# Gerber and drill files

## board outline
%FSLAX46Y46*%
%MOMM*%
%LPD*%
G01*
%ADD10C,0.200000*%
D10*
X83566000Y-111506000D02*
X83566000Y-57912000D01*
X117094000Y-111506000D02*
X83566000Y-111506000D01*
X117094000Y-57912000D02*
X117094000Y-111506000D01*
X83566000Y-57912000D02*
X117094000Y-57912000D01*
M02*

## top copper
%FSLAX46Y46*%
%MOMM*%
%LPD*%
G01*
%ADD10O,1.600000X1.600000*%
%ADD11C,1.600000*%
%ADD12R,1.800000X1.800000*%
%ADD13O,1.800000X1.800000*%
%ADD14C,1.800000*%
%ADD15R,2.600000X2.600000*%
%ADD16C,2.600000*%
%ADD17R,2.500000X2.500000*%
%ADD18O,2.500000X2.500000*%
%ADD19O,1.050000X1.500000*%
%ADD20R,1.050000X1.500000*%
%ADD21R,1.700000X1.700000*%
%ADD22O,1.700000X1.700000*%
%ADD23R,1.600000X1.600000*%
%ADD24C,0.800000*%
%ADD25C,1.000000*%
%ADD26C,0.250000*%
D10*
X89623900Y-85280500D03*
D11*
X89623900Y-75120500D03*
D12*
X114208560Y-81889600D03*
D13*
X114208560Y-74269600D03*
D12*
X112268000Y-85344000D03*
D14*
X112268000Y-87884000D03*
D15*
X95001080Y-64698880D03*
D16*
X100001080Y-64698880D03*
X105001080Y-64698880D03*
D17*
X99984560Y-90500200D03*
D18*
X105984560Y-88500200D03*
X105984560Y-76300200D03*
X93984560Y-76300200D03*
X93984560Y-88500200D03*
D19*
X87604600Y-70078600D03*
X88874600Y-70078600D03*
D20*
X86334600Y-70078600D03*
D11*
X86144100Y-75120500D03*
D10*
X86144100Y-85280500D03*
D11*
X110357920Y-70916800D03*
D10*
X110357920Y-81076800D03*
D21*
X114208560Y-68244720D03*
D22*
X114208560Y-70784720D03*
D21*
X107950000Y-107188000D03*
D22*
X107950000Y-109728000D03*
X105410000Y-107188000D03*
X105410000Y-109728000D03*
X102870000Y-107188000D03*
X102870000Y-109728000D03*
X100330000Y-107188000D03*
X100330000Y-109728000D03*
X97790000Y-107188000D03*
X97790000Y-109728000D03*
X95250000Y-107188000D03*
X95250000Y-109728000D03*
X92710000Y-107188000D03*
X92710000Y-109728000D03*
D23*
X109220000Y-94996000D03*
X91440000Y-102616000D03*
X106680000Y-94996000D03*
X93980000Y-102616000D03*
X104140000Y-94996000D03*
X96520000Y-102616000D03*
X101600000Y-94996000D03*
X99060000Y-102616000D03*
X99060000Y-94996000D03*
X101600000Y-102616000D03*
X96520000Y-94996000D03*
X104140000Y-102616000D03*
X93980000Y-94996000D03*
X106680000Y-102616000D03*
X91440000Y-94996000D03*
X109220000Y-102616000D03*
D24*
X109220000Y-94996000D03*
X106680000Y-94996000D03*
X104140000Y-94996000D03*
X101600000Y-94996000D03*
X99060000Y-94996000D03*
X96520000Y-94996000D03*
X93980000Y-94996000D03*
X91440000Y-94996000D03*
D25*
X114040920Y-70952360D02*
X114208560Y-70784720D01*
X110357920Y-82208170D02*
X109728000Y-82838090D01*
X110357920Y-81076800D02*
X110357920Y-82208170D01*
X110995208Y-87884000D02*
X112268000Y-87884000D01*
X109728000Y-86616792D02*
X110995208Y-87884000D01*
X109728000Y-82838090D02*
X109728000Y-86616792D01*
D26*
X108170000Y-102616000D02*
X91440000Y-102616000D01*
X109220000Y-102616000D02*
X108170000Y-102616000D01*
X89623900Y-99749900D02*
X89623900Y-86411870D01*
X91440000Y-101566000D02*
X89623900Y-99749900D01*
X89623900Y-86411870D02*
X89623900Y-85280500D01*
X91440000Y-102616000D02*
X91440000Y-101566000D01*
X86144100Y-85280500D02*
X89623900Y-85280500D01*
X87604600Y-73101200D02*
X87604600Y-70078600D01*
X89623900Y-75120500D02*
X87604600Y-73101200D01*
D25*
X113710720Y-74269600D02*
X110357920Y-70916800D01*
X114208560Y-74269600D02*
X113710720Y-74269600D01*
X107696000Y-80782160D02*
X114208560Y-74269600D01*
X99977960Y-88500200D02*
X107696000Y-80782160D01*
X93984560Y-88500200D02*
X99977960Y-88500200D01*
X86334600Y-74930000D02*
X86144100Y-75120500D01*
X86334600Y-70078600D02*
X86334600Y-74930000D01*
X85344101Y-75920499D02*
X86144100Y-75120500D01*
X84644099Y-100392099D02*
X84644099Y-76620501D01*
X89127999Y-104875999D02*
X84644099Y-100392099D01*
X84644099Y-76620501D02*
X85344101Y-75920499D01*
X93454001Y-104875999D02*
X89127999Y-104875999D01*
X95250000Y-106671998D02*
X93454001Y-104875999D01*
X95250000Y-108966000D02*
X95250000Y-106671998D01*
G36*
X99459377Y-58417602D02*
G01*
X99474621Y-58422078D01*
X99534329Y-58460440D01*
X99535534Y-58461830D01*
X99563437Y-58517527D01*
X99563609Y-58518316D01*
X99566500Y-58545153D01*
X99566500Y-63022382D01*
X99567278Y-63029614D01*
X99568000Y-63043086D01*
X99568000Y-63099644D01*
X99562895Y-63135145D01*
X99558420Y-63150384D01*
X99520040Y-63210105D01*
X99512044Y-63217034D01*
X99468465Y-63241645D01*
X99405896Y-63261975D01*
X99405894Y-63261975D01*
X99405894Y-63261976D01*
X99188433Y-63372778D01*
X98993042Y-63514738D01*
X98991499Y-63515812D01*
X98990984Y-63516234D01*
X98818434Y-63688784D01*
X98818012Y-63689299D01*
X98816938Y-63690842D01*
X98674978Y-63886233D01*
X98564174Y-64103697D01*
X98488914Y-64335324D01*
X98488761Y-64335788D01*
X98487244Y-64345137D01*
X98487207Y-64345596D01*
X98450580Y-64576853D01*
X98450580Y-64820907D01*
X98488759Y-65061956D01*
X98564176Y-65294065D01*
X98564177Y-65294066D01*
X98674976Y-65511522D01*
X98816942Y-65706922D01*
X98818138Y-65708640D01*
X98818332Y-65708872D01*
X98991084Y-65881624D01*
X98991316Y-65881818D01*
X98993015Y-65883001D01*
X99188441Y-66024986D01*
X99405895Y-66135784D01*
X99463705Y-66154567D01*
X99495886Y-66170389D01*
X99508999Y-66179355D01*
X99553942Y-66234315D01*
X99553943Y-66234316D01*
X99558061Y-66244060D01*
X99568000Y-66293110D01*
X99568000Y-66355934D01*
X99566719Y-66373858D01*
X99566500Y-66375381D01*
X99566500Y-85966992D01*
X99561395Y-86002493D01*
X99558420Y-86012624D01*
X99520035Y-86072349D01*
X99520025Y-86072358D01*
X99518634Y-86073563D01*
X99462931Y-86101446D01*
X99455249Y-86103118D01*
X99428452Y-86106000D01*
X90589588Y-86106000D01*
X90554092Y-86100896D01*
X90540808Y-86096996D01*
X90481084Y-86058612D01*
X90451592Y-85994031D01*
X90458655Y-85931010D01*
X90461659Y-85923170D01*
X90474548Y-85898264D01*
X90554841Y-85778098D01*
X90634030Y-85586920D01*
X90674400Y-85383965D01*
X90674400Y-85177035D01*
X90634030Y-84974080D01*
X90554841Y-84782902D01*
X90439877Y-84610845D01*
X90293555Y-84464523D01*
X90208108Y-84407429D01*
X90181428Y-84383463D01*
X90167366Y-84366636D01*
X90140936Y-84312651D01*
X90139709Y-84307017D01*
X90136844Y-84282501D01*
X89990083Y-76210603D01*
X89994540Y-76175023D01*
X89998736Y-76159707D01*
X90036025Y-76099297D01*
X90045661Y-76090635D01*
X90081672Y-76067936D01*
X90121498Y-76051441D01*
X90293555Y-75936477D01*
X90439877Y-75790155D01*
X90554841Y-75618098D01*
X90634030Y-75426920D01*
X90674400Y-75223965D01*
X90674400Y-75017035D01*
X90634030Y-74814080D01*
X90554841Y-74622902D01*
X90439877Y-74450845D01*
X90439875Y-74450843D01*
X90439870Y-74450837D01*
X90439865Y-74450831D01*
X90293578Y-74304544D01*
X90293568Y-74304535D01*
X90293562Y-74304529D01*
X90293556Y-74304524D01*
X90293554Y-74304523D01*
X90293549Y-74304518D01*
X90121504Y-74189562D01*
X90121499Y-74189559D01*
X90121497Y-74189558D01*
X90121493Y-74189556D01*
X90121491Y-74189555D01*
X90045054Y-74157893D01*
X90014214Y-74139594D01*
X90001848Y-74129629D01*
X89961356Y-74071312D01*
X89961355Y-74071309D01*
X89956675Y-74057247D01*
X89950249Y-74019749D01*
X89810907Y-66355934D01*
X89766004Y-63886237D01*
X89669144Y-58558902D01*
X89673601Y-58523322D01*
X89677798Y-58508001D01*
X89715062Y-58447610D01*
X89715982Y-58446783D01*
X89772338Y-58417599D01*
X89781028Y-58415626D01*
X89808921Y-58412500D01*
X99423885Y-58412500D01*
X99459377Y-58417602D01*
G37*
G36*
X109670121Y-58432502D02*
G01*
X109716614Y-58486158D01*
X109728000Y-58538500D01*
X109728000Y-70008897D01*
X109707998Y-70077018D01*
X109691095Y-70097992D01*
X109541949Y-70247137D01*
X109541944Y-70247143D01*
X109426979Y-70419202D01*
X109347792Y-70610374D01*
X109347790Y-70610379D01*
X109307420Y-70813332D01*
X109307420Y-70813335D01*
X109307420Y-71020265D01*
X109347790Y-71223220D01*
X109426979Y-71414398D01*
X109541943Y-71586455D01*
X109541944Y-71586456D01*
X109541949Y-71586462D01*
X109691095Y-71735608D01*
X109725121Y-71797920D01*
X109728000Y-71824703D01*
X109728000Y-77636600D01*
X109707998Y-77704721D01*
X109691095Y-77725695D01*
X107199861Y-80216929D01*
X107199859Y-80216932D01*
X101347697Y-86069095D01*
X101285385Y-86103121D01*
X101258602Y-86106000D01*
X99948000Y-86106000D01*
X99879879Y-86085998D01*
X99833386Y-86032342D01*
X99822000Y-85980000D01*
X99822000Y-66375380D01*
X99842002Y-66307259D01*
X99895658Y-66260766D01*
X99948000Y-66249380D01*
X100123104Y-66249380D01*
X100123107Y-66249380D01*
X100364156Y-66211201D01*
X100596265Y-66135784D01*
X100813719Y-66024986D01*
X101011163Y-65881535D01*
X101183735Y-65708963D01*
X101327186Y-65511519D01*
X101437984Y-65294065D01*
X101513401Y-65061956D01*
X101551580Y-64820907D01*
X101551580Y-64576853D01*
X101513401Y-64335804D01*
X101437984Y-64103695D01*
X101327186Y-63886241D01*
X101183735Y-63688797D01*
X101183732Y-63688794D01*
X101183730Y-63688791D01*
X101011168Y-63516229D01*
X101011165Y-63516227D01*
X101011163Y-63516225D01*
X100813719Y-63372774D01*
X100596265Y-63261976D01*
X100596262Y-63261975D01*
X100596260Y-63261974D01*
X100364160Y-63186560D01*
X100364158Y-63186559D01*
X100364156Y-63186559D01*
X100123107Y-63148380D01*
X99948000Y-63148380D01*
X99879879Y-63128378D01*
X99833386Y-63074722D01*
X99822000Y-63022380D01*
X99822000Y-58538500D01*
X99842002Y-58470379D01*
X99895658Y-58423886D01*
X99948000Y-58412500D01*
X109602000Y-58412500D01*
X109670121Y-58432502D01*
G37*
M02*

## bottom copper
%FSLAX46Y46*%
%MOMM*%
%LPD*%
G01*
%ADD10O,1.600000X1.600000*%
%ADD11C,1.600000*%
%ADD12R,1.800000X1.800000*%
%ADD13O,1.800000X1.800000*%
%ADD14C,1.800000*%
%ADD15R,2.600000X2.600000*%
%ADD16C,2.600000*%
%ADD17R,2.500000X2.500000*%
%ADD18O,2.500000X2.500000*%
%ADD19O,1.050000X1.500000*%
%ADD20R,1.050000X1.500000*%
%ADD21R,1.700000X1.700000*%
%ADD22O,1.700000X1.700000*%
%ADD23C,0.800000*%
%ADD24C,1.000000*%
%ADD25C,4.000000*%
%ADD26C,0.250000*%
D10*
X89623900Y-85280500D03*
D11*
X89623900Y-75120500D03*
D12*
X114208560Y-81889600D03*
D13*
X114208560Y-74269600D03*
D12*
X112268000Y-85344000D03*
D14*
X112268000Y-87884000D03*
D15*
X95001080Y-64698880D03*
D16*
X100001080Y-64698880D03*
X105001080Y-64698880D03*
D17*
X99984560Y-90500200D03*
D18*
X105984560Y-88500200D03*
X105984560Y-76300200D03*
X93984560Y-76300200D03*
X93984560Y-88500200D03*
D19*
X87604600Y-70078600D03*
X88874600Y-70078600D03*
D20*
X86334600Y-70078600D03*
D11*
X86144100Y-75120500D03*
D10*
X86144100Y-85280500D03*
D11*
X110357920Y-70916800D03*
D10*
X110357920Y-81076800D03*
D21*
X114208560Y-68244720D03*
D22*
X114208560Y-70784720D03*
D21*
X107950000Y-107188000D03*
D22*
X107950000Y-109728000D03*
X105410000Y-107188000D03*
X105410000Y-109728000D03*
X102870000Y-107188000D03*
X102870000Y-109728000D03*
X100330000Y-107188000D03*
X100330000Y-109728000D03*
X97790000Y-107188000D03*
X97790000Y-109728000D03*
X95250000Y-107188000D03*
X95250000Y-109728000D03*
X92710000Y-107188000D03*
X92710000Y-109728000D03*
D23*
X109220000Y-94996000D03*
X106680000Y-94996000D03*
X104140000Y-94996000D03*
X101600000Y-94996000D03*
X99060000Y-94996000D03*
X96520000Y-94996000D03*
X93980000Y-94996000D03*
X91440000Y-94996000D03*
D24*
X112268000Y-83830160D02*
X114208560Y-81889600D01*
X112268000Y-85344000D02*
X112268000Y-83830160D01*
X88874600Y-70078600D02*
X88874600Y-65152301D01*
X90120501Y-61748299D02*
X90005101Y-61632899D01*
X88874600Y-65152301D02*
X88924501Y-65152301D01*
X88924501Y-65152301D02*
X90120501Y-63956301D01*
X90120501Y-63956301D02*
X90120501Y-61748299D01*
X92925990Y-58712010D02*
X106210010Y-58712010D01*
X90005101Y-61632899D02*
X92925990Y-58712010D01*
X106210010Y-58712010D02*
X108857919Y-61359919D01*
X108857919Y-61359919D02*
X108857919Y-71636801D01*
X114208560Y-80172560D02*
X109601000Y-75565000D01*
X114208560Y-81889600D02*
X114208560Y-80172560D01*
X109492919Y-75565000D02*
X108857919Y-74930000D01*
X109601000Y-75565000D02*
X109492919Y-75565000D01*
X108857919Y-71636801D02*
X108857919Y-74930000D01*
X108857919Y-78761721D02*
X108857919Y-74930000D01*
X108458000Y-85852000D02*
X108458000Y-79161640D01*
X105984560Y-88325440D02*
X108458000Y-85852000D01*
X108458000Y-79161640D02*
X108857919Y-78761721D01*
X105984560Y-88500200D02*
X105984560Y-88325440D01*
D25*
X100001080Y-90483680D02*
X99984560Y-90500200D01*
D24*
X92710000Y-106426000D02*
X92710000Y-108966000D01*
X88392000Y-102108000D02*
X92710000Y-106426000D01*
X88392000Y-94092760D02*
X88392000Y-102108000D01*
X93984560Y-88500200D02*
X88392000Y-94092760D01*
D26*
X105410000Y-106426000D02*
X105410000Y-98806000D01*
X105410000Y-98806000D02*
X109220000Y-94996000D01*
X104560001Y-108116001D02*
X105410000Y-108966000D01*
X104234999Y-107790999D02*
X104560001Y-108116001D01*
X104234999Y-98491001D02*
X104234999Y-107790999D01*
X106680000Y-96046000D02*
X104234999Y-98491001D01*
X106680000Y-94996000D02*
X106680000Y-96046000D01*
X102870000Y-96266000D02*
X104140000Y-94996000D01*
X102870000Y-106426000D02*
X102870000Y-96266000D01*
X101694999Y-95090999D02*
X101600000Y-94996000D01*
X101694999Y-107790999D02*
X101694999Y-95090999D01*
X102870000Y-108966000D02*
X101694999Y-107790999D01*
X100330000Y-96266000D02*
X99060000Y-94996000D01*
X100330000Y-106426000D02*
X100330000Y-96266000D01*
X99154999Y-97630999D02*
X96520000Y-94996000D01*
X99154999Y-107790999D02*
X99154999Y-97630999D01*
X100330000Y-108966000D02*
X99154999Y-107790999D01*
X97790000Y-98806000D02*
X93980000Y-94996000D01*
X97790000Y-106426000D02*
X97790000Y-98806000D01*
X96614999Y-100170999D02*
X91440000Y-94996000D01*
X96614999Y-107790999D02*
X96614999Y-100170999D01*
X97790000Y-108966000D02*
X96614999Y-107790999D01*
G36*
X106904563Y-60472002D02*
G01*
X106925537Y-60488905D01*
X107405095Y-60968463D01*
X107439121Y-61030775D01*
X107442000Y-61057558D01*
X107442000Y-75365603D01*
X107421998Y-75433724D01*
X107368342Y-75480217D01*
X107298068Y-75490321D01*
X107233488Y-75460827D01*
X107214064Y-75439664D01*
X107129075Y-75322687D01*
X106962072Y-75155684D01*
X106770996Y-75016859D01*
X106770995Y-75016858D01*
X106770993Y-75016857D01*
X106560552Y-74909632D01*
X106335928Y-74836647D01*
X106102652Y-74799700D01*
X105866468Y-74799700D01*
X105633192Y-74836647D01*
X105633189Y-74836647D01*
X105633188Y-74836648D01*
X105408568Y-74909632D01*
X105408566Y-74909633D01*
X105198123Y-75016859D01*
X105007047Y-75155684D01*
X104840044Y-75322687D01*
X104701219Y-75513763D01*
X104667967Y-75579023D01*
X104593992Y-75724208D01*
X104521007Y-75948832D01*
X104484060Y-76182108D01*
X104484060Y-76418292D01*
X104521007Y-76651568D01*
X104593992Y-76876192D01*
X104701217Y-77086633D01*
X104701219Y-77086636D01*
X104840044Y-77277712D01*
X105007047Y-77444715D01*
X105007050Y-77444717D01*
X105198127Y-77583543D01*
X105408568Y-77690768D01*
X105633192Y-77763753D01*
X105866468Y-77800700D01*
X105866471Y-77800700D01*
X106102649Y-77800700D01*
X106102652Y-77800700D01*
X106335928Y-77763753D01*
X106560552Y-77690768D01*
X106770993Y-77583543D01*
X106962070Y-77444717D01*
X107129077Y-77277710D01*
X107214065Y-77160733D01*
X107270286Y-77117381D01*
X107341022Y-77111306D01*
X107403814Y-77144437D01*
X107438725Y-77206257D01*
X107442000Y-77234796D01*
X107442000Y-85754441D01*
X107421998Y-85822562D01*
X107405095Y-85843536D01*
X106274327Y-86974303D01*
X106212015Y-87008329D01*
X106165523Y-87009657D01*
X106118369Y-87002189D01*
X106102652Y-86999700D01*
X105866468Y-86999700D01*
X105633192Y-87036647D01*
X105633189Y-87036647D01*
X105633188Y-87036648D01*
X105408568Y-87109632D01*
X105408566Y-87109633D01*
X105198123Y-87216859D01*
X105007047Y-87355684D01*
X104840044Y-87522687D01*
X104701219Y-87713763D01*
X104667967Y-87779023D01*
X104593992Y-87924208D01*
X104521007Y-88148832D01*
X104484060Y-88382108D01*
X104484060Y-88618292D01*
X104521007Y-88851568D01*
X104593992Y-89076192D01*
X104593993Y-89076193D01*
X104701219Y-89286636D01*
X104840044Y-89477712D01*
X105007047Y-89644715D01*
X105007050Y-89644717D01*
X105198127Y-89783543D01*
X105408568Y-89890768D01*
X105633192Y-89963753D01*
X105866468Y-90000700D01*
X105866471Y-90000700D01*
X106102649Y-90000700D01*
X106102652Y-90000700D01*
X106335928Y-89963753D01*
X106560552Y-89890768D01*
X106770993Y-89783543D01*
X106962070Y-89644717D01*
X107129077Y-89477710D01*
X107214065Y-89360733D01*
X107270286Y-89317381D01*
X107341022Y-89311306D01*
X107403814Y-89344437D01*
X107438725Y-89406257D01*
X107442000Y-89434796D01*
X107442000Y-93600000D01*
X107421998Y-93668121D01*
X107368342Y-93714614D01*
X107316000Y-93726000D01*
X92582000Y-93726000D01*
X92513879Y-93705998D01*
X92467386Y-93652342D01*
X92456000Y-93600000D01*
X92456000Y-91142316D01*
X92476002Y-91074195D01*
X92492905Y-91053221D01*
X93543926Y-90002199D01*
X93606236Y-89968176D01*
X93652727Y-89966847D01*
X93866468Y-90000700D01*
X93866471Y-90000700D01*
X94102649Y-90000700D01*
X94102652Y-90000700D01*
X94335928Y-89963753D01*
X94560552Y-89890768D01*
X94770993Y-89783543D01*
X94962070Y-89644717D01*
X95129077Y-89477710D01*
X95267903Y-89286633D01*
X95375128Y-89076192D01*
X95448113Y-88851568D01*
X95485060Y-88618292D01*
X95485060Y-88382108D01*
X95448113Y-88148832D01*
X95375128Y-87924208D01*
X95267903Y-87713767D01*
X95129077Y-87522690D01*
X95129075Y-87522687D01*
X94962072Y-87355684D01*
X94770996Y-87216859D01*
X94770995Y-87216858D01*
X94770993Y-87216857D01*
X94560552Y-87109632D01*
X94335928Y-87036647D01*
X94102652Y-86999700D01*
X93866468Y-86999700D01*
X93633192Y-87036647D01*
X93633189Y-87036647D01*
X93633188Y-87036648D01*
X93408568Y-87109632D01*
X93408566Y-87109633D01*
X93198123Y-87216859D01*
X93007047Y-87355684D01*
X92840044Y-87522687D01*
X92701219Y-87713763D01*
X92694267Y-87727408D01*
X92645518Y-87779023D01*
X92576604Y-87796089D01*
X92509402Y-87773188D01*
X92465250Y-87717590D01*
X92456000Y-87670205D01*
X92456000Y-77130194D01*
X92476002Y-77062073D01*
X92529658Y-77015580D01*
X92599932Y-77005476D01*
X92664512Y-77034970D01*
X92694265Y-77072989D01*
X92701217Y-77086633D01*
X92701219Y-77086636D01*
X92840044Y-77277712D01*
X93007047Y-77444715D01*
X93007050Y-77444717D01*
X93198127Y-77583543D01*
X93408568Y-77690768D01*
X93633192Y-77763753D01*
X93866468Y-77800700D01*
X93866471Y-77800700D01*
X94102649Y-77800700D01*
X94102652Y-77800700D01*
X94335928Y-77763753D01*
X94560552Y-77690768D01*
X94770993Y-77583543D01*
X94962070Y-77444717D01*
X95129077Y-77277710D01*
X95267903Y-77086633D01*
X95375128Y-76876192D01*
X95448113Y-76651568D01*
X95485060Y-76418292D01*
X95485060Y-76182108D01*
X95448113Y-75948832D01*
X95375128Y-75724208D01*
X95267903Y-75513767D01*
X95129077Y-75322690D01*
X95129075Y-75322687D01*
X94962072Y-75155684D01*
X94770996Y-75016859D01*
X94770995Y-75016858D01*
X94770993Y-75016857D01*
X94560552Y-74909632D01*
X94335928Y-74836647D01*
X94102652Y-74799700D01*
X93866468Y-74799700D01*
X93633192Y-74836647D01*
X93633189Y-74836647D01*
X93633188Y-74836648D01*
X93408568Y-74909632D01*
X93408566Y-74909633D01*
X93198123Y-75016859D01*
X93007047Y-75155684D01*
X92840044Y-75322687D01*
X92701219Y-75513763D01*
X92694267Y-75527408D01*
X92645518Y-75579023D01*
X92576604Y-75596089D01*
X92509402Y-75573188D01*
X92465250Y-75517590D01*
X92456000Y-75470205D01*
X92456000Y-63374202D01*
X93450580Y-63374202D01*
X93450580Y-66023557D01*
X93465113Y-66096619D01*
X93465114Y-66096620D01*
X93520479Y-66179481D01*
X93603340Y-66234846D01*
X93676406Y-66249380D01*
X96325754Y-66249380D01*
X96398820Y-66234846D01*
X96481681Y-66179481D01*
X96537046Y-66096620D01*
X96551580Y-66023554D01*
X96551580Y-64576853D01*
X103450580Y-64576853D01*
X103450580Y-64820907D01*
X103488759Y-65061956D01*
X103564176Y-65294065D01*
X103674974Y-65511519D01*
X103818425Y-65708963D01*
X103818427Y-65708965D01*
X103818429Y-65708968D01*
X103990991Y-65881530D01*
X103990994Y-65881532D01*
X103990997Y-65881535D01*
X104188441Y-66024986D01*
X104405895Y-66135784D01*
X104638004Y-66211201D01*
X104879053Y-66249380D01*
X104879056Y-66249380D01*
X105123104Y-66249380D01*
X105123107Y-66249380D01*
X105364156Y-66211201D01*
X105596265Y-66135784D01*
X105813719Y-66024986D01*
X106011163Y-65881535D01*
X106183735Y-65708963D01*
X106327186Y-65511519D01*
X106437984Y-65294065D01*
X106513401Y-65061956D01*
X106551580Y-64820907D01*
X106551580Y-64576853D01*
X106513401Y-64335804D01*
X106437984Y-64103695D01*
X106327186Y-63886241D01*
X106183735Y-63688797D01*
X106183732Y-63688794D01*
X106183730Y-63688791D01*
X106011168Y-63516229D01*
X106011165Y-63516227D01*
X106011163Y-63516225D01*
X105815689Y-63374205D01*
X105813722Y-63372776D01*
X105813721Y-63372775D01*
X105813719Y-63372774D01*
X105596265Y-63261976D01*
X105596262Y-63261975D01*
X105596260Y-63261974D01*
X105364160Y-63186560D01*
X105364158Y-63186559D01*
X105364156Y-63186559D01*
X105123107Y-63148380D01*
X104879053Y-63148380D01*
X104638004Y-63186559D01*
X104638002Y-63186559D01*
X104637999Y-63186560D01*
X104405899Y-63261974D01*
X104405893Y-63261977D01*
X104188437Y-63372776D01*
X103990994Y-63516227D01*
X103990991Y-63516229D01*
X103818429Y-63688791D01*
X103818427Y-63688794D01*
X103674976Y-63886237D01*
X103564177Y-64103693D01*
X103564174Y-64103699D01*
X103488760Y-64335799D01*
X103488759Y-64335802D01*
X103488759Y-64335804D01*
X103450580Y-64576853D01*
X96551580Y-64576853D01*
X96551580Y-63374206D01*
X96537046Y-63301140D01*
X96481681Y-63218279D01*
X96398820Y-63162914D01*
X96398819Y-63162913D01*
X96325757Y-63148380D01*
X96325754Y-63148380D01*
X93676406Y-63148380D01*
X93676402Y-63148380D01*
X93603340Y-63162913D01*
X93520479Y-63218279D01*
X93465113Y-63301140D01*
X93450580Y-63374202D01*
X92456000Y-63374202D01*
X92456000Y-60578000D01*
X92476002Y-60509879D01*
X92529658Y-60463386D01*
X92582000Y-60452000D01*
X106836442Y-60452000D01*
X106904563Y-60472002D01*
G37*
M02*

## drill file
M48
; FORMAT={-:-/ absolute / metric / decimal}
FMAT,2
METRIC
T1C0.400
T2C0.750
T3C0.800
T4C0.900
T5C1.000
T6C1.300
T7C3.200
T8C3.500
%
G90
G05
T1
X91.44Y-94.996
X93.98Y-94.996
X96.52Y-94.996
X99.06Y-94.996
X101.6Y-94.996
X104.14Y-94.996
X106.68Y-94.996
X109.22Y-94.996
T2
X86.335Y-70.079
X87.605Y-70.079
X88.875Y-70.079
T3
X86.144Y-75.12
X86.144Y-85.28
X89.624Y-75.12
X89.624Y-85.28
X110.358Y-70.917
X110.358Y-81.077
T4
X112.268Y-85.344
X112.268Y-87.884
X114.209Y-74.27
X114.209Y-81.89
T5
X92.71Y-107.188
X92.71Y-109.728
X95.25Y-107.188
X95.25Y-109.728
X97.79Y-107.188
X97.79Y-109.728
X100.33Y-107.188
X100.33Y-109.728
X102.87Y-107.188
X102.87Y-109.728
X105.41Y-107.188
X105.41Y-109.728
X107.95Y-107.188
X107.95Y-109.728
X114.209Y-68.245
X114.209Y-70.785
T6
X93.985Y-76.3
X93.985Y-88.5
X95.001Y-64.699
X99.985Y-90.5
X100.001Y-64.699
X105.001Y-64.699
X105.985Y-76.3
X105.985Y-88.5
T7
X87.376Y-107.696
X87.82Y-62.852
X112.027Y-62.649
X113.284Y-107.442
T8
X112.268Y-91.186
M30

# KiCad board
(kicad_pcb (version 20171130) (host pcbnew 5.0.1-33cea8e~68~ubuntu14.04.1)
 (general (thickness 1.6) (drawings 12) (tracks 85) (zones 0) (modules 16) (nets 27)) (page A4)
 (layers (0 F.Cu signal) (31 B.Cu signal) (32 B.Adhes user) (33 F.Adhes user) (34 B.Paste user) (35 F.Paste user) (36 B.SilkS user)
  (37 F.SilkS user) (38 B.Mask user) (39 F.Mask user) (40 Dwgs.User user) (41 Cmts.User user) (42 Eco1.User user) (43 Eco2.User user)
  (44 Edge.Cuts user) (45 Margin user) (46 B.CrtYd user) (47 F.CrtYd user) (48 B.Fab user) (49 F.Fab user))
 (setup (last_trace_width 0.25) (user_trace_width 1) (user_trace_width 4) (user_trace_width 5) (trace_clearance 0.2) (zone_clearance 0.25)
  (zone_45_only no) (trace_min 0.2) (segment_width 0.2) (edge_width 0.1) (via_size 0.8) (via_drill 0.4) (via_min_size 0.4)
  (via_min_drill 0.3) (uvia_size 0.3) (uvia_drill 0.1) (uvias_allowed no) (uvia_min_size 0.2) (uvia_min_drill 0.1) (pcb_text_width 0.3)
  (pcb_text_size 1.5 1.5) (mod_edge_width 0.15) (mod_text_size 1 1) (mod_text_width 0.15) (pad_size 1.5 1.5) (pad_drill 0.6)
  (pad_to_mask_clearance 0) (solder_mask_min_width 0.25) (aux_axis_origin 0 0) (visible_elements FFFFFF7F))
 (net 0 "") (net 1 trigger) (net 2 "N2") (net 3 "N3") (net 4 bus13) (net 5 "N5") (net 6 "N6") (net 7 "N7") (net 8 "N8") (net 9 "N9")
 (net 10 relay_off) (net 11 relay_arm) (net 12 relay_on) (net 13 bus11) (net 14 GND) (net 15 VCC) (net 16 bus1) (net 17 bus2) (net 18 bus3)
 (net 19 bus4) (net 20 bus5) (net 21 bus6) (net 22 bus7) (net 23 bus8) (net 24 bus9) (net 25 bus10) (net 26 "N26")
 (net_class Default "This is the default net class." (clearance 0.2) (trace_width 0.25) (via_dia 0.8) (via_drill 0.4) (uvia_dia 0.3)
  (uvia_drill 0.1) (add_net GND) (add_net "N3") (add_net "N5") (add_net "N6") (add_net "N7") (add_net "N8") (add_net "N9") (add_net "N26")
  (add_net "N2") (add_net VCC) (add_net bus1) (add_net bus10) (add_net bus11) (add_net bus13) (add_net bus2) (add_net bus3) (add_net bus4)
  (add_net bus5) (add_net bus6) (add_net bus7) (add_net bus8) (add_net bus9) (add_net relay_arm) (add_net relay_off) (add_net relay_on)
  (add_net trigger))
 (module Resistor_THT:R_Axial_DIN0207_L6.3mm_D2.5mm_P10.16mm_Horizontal (layer F.Cu) (at 89.6239 75.1205 270)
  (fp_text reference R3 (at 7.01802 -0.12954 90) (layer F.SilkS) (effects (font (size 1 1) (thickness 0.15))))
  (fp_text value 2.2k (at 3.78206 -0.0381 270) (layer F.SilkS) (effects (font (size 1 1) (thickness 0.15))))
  (pad 2 thru_hole oval (at 10.16 0 270) (size 1.6 1.6) (drill 0.8) (layers *.Cu *.Mask) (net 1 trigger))
  (pad 1 thru_hole circle (at 0 0 270) (size 1.6 1.6) (drill 0.8) (layers *.Cu *.Mask) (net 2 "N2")))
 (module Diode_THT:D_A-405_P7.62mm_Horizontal (layer F.Cu) (at 114.20856 81.8896 90)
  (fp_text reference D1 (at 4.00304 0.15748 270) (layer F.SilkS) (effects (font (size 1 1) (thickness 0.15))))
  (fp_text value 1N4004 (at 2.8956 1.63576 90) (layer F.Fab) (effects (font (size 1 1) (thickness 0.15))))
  (pad 1 thru_hole rect (at 0 0 90) (size 1.8 1.8) (drill 0.9) (layers *.Cu *.Mask) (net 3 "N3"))
  (pad 2 thru_hole oval (at 7.62 0 90) (size 1.8 1.8) (drill 0.9) (layers *.Cu *.Mask) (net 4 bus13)))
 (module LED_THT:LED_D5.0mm (layer B.Cu) (at 112.268 85.344 270)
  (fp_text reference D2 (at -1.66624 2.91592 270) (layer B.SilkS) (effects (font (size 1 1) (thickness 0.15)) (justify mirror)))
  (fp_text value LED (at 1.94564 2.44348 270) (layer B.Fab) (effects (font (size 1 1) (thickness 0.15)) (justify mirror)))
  (pad 1 thru_hole rect (at 0 0 270) (size 1.8 1.8) (drill 0.9) (layers *.Cu *.Mask) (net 3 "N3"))
  (pad 2 thru_hole circle (at 2.54 0 270) (size 1.8 1.8) (drill 0.9) (layers *.Cu *.Mask) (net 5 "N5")))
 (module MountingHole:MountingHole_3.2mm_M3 (layer F.Cu) (at 87.376 107.696)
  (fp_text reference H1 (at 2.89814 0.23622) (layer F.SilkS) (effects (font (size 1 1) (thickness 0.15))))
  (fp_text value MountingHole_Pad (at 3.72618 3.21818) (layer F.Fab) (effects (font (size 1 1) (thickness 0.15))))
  (pad 1 np_thru_hole circle (at 0 0) (size 3.2 3.2) (drill 3.2) (layers *.Cu *.Mask) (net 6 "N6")))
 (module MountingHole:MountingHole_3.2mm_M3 (layer F.Cu) (at 113.284 107.442)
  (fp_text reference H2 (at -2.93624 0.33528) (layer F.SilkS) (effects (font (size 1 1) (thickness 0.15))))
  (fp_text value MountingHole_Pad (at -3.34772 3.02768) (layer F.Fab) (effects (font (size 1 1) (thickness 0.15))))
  (pad 1 np_thru_hole circle (at 0 0) (size 3.2 3.2) (drill 3.2) (layers *.Cu *.Mask) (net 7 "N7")))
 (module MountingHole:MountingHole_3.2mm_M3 (layer F.Cu) (at 112.0267 62.6491)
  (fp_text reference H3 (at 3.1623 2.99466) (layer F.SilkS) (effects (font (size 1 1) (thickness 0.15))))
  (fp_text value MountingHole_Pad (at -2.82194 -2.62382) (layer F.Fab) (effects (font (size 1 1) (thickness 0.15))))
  (pad 1 np_thru_hole circle (at 0 0) (size 3.2 3.2) (drill 3.2) (layers *.Cu *.Mask) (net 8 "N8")))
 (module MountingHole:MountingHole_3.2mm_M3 (layer F.Cu) (at 87.8205 62.8523)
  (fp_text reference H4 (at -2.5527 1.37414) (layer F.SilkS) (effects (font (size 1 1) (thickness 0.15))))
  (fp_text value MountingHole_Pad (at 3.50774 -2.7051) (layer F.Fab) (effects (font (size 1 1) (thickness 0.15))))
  (pad 1 np_thru_hole circle (at 0 0) (size 3.2 3.2) (drill 3.2) (layers *.Cu *.Mask) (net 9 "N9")))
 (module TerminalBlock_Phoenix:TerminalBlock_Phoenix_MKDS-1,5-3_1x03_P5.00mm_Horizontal (layer F.Cu) (at 95.00108 64.69888)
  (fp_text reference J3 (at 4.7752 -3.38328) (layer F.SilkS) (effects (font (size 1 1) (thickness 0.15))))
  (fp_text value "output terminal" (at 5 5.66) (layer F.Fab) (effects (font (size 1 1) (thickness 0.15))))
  (pad 1 thru_hole rect (at 0 0) (size 2.6 2.6) (drill 1.3) (layers *.Cu *.Mask) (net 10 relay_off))
  (pad 2 thru_hole circle (at 5 0) (size 2.6 2.6) (drill 1.3) (layers *.Cu *.Mask) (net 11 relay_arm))
  (pad 3 thru_hole circle (at 10 0) (size 2.6 2.6) (drill 1.3) (layers *.Cu *.Mask) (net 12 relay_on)))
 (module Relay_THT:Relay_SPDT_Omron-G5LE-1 (layer F.Cu) (at 99.98456 90.5002 180)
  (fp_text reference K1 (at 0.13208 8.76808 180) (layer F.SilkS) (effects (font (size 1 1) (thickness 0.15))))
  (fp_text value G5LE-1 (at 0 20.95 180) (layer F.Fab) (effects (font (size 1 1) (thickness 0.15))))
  (pad 1 thru_hole rect (at 0 0 180) (size 2.5 2.5) (drill 1.3) (layers *.Cu *.Mask) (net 11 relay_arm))
  (pad 2 thru_hole oval (at -6 2 180) (size 2.5 2.5) (drill 1.3) (layers *.Cu *.Mask) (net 3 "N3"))
  (pad 3 thru_hole oval (at -6 14.2 180) (size 2.5 2.5) (drill 1.3) (layers *.Cu *.Mask) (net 12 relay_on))
  (pad 4 thru_hole oval (at 6 14.2 180) (size 2.5 2.5) (drill 1.3) (layers *.Cu *.Mask) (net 10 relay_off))
  (pad 5 thru_hole oval (at 6 2 180) (size 2.5 2.5) (drill 1.3) (layers *.Cu *.Mask) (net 4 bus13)))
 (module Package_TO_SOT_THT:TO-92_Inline (layer F.Cu) (at 86.3346 70.0786)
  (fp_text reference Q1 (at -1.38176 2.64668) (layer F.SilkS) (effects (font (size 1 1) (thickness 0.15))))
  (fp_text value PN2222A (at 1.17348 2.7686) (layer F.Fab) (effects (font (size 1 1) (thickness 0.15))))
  (pad 2 thru_hole oval (at 1.27 0) (size 1.05 1.5) (drill 0.75) (layers *.Cu *.Mask) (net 2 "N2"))
  (pad 3 thru_hole oval (at 2.54 0) (size 1.05 1.5) (drill 0.75) (layers *.Cu *.Mask) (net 3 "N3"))
  (pad 1 thru_hole rect (at 0 0) (size 1.05 1.5) (drill 0.75) (layers *.Cu *.Mask) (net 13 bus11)))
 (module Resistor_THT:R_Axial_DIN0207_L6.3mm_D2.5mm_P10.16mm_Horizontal (layer F.Cu) (at 86.1441 75.1205 270)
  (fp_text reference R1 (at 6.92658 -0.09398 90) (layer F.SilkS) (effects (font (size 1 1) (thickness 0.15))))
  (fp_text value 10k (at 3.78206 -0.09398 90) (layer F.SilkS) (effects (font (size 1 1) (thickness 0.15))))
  (pad 1 thru_hole circle (at 0 0 270) (size 1.6 1.6) (drill 0.8) (layers *.Cu *.Mask) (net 13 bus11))
  (pad 2 thru_hole oval (at 10.16 0 270) (size 1.6 1.6) (drill 0.8) (layers *.Cu *.Mask) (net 1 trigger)))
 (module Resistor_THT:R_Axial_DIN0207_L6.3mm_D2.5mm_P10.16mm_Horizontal (layer F.Cu) (at 110.35792 70.9168 270)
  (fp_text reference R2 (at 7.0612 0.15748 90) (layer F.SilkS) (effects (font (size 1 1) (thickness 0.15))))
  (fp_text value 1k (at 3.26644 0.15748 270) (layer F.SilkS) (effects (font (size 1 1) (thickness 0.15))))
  (pad 1 thru_hole circle (at 0 0 270) (size 1.6 1.6) (drill 0.8) (layers *.Cu *.Mask) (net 4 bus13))
  (pad 2 thru_hole oval (at 10.16 0 270) (size 1.6 1.6) (drill 0.8) (layers *.Cu *.Mask) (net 5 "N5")))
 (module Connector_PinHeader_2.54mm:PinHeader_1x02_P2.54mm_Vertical (layer F.Cu) (at 114.20856 68.24472)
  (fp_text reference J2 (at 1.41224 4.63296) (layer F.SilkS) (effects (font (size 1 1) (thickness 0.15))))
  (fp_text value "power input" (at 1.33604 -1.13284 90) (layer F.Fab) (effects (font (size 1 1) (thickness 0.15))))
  (pad 1 thru_hole rect (at 0 0) (size 1.7 1.7) (drill 1) (layers *.Cu *.Mask) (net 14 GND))
  (pad 2 thru_hole oval (at 0 2.54) (size 1.7 1.7) (drill 1) (layers *.Cu *.Mask) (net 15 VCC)))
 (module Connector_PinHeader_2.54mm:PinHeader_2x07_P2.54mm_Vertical (layer F.Cu) (at 107.95 107.188 270)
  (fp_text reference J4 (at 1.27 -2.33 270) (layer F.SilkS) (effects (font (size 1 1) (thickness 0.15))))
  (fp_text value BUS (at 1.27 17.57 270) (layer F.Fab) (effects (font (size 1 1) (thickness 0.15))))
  (pad 1 thru_hole rect (at 0 0 270) (size 1.7 1.7) (drill 1) (layers *.Cu *.Mask) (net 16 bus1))
  (pad 2 thru_hole oval (at 2.54 0 270) (size 1.7 1.7) (drill 1) (layers *.Cu *.Mask) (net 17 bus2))
  (pad 3 thru_hole oval (at 0 2.54 270) (size 1.7 1.7) (drill 1) (layers *.Cu *.Mask) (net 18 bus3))
  (pad 4 thru_hole oval (at 2.54 2.54 270) (size 1.7 1.7) (drill 1) (layers *.Cu *.Mask) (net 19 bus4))
  (pad 5 thru_hole oval (at 0 5.08 270) (size 1.7 1.7) (drill 1) (layers *.Cu *.Mask) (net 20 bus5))
  (pad 6 thru_hole oval (at 2.54 5.08 270) (size 1.7 1.7) (drill 1) (layers *.Cu *.Mask) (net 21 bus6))
  (pad 7 thru_hole oval (at 0 7.62 270) (size 1.7 1.7) (drill 1) (layers *.Cu *.Mask) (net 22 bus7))
  (pad 8 thru_hole oval (at 2.54 7.62 270) (size 1.7 1.7) (drill 1) (layers *.Cu *.Mask) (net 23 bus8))
  (pad 9 thru_hole oval (at 0 10.16 270) (size 1.7 1.7) (drill 1) (layers *.Cu *.Mask) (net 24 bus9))
  (pad 10 thru_hole oval (at 2.54 10.16 270) (size 1.7 1.7) (drill 1) (layers *.Cu *.Mask) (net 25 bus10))
  (pad 11 thru_hole oval (at 0 12.7 270) (size 1.7 1.7) (drill 1) (layers *.Cu *.Mask) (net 13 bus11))
  (pad 12 thru_hole oval (at 2.54 12.7 270) (size 1.7 1.7) (drill 1) (layers *.Cu *.Mask) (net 13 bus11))
  (pad 13 thru_hole oval (at 0 15.24 270) (size 1.7 1.7) (drill 1) (layers *.Cu *.Mask) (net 4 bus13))
  (pad 14 thru_hole oval (at 2.54 15.24 270) (size 1.7 1.7) (drill 1) (layers *.Cu *.Mask) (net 4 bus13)))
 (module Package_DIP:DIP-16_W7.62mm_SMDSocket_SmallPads (layer F.Cu) (at 100.33 98.806 270)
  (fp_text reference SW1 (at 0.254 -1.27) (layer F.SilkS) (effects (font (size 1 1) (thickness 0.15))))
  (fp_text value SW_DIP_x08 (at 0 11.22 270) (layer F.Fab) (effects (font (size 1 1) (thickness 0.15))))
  (pad 1 smd rect (at -3.81 -8.89 270) (size 1.6 1.6) (layers F.Cu F.Paste F.Mask) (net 18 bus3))
  (pad 9 smd rect (at 3.81 8.89 270) (size 1.6 1.6) (layers F.Cu F.Paste F.Mask) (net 1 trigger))
  (pad 2 smd rect (at -3.81 -6.35 270) (size 1.6 1.6) (layers F.Cu F.Paste F.Mask) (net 19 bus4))
  (pad 10 smd rect (at 3.81 6.35 270) (size 1.6 1.6) (layers F.Cu F.Paste F.Mask) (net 1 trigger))
  (pad 3 smd rect (at -3.81 -3.81 270) (size 1.6 1.6) (layers F.Cu F.Paste F.Mask) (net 20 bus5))
  (pad 11 smd rect (at 3.81 3.81 270) (size 1.6 1.6) (layers F.Cu F.Paste F.Mask) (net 1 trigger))
  (pad 4 smd rect (at -3.81 -1.27 270) (size 1.6 1.6) (layers F.Cu F.Paste F.Mask) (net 21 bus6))
  (pad 12 smd rect (at 3.81 1.27 270) (size 1.6 1.6) (layers F.Cu F.Paste F.Mask) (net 1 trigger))
  (pad 5 smd rect (at -3.81 1.27 270) (size 1.6 1.6) (layers F.Cu F.Paste F.Mask) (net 22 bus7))
  (pad 13 smd rect (at 3.81 -1.27 270) (size 1.6 1.6) (layers F.Cu F.Paste F.Mask) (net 1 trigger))
  (pad 6 smd rect (at -3.81 3.81 270) (size 1.6 1.6) (layers F.Cu F.Paste F.Mask) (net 23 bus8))
  (pad 14 smd rect (at 3.81 -3.81 270) (size 1.6 1.6) (layers F.Cu F.Paste F.Mask) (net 1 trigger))
  (pad 7 smd rect (at -3.81 6.35 270) (size 1.6 1.6) (layers F.Cu F.Paste F.Mask) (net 24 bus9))
  (pad 15 smd rect (at 3.81 -6.35 270) (size 1.6 1.6) (layers F.Cu F.Paste F.Mask) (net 1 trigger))
  (pad 8 smd rect (at -3.81 8.89 270) (size 1.6 1.6) (layers F.Cu F.Paste F.Mask) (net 25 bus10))
  (pad 16 smd rect (at 3.81 -8.89 270) (size 1.6 1.6) (layers F.Cu F.Paste F.Mask) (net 1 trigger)))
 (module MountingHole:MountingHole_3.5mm (layer F.Cu) (at 112.268 91.186)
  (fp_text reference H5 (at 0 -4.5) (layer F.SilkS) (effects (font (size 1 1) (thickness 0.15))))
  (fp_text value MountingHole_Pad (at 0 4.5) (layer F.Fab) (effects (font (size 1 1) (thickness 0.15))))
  (pad 1 np_thru_hole circle (at 0 0) (size 3.5 3.5) (drill 3.5) (layers *.Cu *.Mask) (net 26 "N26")))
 (gr_line (start 83.566 111.506) (end 83.566 57.912) (layer Edge.Cuts) (width 0.2))
 (gr_line (start 117.094 111.506) (end 83.566 111.506) (layer Edge.Cuts) (width 0.2))
 (gr_line (start 117.094 57.912) (end 117.094 111.506) (layer Edge.Cuts) (width 0.2))
 (gr_line (start 83.566 57.912) (end 117.094 57.912) (layer Edge.Cuts) (width 0.2))
 (segment (start 112.268 83.83016) (end 114.20856 81.8896) (width 1) (layer B.Cu) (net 3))
 (segment (start 112.268 85.344) (end 112.268 83.83016) (width 1) (layer B.Cu) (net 3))
 (segment (start 88.8746 70.0786) (end 88.8746 65.152301) (width 1) (layer B.Cu) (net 3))
 (segment (start 90.120501 61.748299) (end 90.005101 61.632899) (width 1) (layer B.Cu) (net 3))
 (segment (start 88.8746 65.152301) (end 88.924501 65.152301) (width 1) (layer B.Cu) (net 3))
 (segment (start 88.924501 65.152301) (end 90.120501 63.956301) (width 1) (layer B.Cu) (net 3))
 (segment (start 90.120501 63.956301) (end 90.120501 61.748299) (width 1) (layer B.Cu) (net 3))
 (segment (start 92.92599 58.71201) (end 106.21001 58.71201) (width 1) (layer B.Cu) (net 3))
 (segment (start 90.005101 61.632899) (end 92.92599 58.71201) (width 1) (layer B.Cu) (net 3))
 (segment (start 106.21001 58.71201) (end 108.857919 61.359919) (width 1) (layer B.Cu) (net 3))
 (segment (start 108.857919 61.359919) (end 108.857919 71.636801) (width 1) (layer B.Cu) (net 3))
 (segment (start 114.20856 80.17256) (end 109.601 75.565) (width 1) (layer B.Cu) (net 3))
 (segment (start 114.20856 81.8896) (end 114.20856 80.17256) (width 1) (layer B.Cu) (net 3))
 (segment (start 109.492919 75.565) (end 108.857919 74.93) (width 1) (layer B.Cu) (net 3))
 (segment (start 109.601 75.565) (end 109.492919 75.565) (width 1) (layer B.Cu) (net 3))
 (segment (start 108.857919 71.636801) (end 108.857919 74.93) (width 1) (layer B.Cu) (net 3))
 (segment (start 108.857919 78.761721) (end 108.857919 74.93) (width 1) (layer B.Cu) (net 3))
 (segment (start 108.458 85.852) (end 108.458 79.16164) (width 1) (layer B.Cu) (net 3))
 (segment (start 105.98456 88.32544) (end 108.458 85.852) (width 1) (layer B.Cu) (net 3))
 (segment (start 108.458 79.16164) (end 108.857919 78.761721) (width 1) (layer B.Cu) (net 3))
 (segment (start 105.98456 88.5002) (end 105.98456 88.32544) (width 1) (layer B.Cu) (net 3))
 (segment (start 114.04092 70.95236) (end 114.20856 70.78472) (width 1) (layer F.Cu) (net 15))
 (segment (start 110.35792 82.20817) (end 109.728 82.83809) (width 1) (layer F.Cu) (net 5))
 (segment (start 110.35792 81.0768) (end 110.35792 82.20817) (width 1) (layer F.Cu) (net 5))
 (segment (start 110.995208 87.884) (end 112.268 87.884) (width 1) (layer F.Cu) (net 5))
 (segment (start 109.728 86.616792) (end 110.995208 87.884) (width 1) (layer F.Cu) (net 5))
 (segment (start 109.728 82.83809) (end 109.728 86.616792) (width 1) (layer F.Cu) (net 5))
 (segment (start 108.17 102.616) (end 91.44 102.616) (width 0.25) (layer F.Cu) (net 1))
 (segment (start 109.22 102.616) (end 108.17 102.616) (width 0.25) (layer F.Cu) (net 1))
 (segment (start 89.6239 99.7499) (end 89.6239 86.41187) (width 0.25) (layer F.Cu) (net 1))
 (segment (start 91.44 101.566) (end 89.6239 99.7499) (width 0.25) (layer F.Cu) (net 1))
 (segment (start 89.6239 86.41187) (end 89.6239 85.2805) (width 0.25) (layer F.Cu) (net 1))
 (segment (start 91.44 102.616) (end 91.44 101.566) (width 0.25) (layer F.Cu) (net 1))
 (segment (start 86.1441 85.2805) (end 89.6239 85.2805) (width 0.25) (layer F.Cu) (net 1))
 (segment (start 100.00108 90.48368) (end 99.98456 90.5002) (width 4) (layer B.Cu) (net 11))
 (segment (start 87.6046 73.1012) (end 87.6046 70.0786) (width 0.25) (layer F.Cu) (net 2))
 (segment (start 89.6239 75.1205) (end 87.6046 73.1012) (width 0.25) (layer F.Cu) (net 2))
 (segment (start 113.71072 74.2696) (end 110.35792 70.9168) (width 1) (layer F.Cu) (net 4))
 (segment (start 114.20856 74.2696) (end 113.71072 74.2696) (width 1) (layer F.Cu) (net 4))
 (segment (start 107.696 80.78216) (end 114.20856 74.2696) (width 1) (layer F.Cu) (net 4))
 (segment (start 99.97796 88.5002) (end 107.696 80.78216) (width 1) (layer F.Cu) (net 4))
 (segment (start 93.98456 88.5002) (end 99.97796 88.5002) (width 1) (layer F.Cu) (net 4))
 (segment (start 92.71 106.426) (end 92.71 108.966) (width 1) (layer B.Cu) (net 4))
 (segment (start 88.392 102.108) (end 92.71 106.426) (width 1) (layer B.Cu) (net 4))
 (segment (start 88.392 94.09276) (end 88.392 102.108) (width 1) (layer B.Cu) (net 4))
 (segment (start 93.98456 88.5002) (end 88.392 94.09276) (width 1) (layer B.Cu) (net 4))
 (via (at 109.22 94.996) (size 0.8) (drill 0.4) (layers F.Cu B.Cu) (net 18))
 (segment (start 105.41 106.426) (end 105.41 98.806) (width 0.25) (layer B.Cu) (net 18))
 (segment (start 105.41 98.806) (end 109.22 94.996) (width 0.25) (layer B.Cu) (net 18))
 (via (at 106.68 94.996) (size 0.8) (drill 0.4) (layers F.Cu B.Cu) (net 19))
 (segment (start 104.560001 108.116001) (end 105.41 108.966) (width 0.25) (layer B.Cu) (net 19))
 (segment (start 104.234999 107.790999) (end 104.560001 108.116001) (width 0.25) (layer B.Cu) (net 19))
 (segment (start 104.234999 98.491001) (end 104.234999 107.790999) (width 0.25) (layer B.Cu) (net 19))
 (segment (start 106.68 96.046) (end 104.234999 98.491001) (width 0.25) (layer B.Cu) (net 19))
 (segment (start 106.68 94.996) (end 106.68 96.046) (width 0.25) (layer B.Cu) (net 19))
 (via (at 104.14 94.996) (size 0.8) (drill 0.4) (layers F.Cu B.Cu) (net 20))
 (segment (start 102.87 96.266) (end 104.14 94.996) (width 0.25) (layer B.Cu) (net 20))
 (segment (start 102.87 106.426) (end 102.87 96.266) (width 0.25) (layer B.Cu) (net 20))
 (via (at 101.6 94.996) (size 0.8) (drill 0.4) (layers F.Cu B.Cu) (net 21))
 (segment (start 101.694999 95.090999) (end 101.6 94.996) (width 0.25) (layer B.Cu) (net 21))
 (segment (start 101.694999 107.790999) (end 101.694999 95.090999) (width 0.25) (layer B.Cu) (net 21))
 (segment (start 102.87 108.966) (end 101.694999 107.790999) (width 0.25) (layer B.Cu) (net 21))
 (via (at 99.06 94.996) (size 0.8) (drill 0.4) (layers F.Cu B.Cu) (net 22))
 (segment (start 100.33 96.266) (end 99.06 94.996) (width 0.25) (layer B.Cu) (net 22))
 (segment (start 100.33 106.426) (end 100.33 96.266) (width 0.25) (layer B.Cu) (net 22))
 (segment (start 99.154999 97.630999) (end 96.52 94.996) (width 0.25) (layer B.Cu) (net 23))
 (via (at 96.52 94.996) (size 0.8) (drill 0.4) (layers F.Cu B.Cu) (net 23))
 (segment (start 99.154999 107.790999) (end 99.154999 97.630999) (width 0.25) (layer B.Cu) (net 23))
 (segment (start 100.33 108.966) (end 99.154999 107.790999) (width 0.25) (layer B.Cu) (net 23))
 (via (at 93.98 94.996) (size 0.8) (drill 0.4) (layers F.Cu B.Cu) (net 24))
 (segment (start 97.79 98.806) (end 93.98 94.996) (width 0.25) (layer B.Cu) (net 24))
 (segment (start 97.79 106.426) (end 97.79 98.806) (width 0.25) (layer B.Cu) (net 24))
 (via (at 91.44 94.996) (size 0.8) (drill 0.4) (layers F.Cu B.Cu) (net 25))
 (segment (start 96.614999 100.170999) (end 91.44 94.996) (width 0.25) (layer B.Cu) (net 25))
 (segment (start 96.614999 107.790999) (end 96.614999 100.170999) (width 0.25) (layer B.Cu) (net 25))
 (segment (start 97.79 108.966) (end 96.614999 107.790999) (width 0.25) (layer B.Cu) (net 25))
 (segment (start 86.3346 74.93) (end 86.1441 75.1205) (width 1) (layer F.Cu) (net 13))
 (segment (start 86.3346 70.0786) (end 86.3346 74.93) (width 1) (layer F.Cu) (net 13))
 (segment (start 85.344101 75.920499) (end 86.1441 75.1205) (width 1) (layer F.Cu) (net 13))
 (segment (start 84.644099 100.392099) (end 84.644099 76.620501) (width 1) (layer F.Cu) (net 13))
 (segment (start 89.127999 104.875999) (end 84.644099 100.392099) (width 1) (layer F.Cu) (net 13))
 (segment (start 84.644099 76.620501) (end 85.344101 75.920499) (width 1) (layer F.Cu) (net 13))
 (segment (start 93.454001 104.875999) (end 89.127999 104.875999) (width 1) (layer F.Cu) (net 13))
 (segment (start 95.25 106.671998) (end 93.454001 104.875999) (width 1) (layer F.Cu) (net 13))
 (segment (start 95.25 108.966) (end 95.25 106.671998) (width 1) (layer F.Cu) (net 13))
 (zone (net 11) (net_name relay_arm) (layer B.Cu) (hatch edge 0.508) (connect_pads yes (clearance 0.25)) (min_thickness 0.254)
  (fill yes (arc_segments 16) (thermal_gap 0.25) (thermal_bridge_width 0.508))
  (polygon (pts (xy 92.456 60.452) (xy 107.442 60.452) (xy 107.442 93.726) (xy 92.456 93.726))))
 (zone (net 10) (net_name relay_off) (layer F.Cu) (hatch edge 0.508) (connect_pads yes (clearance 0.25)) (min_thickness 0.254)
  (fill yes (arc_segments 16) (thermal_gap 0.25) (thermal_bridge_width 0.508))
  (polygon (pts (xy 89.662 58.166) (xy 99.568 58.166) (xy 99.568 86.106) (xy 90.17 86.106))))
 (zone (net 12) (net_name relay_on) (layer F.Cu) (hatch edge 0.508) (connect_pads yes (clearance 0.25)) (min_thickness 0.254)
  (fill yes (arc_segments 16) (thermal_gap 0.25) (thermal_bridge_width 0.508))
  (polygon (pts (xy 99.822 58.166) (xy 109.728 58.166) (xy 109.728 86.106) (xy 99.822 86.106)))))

